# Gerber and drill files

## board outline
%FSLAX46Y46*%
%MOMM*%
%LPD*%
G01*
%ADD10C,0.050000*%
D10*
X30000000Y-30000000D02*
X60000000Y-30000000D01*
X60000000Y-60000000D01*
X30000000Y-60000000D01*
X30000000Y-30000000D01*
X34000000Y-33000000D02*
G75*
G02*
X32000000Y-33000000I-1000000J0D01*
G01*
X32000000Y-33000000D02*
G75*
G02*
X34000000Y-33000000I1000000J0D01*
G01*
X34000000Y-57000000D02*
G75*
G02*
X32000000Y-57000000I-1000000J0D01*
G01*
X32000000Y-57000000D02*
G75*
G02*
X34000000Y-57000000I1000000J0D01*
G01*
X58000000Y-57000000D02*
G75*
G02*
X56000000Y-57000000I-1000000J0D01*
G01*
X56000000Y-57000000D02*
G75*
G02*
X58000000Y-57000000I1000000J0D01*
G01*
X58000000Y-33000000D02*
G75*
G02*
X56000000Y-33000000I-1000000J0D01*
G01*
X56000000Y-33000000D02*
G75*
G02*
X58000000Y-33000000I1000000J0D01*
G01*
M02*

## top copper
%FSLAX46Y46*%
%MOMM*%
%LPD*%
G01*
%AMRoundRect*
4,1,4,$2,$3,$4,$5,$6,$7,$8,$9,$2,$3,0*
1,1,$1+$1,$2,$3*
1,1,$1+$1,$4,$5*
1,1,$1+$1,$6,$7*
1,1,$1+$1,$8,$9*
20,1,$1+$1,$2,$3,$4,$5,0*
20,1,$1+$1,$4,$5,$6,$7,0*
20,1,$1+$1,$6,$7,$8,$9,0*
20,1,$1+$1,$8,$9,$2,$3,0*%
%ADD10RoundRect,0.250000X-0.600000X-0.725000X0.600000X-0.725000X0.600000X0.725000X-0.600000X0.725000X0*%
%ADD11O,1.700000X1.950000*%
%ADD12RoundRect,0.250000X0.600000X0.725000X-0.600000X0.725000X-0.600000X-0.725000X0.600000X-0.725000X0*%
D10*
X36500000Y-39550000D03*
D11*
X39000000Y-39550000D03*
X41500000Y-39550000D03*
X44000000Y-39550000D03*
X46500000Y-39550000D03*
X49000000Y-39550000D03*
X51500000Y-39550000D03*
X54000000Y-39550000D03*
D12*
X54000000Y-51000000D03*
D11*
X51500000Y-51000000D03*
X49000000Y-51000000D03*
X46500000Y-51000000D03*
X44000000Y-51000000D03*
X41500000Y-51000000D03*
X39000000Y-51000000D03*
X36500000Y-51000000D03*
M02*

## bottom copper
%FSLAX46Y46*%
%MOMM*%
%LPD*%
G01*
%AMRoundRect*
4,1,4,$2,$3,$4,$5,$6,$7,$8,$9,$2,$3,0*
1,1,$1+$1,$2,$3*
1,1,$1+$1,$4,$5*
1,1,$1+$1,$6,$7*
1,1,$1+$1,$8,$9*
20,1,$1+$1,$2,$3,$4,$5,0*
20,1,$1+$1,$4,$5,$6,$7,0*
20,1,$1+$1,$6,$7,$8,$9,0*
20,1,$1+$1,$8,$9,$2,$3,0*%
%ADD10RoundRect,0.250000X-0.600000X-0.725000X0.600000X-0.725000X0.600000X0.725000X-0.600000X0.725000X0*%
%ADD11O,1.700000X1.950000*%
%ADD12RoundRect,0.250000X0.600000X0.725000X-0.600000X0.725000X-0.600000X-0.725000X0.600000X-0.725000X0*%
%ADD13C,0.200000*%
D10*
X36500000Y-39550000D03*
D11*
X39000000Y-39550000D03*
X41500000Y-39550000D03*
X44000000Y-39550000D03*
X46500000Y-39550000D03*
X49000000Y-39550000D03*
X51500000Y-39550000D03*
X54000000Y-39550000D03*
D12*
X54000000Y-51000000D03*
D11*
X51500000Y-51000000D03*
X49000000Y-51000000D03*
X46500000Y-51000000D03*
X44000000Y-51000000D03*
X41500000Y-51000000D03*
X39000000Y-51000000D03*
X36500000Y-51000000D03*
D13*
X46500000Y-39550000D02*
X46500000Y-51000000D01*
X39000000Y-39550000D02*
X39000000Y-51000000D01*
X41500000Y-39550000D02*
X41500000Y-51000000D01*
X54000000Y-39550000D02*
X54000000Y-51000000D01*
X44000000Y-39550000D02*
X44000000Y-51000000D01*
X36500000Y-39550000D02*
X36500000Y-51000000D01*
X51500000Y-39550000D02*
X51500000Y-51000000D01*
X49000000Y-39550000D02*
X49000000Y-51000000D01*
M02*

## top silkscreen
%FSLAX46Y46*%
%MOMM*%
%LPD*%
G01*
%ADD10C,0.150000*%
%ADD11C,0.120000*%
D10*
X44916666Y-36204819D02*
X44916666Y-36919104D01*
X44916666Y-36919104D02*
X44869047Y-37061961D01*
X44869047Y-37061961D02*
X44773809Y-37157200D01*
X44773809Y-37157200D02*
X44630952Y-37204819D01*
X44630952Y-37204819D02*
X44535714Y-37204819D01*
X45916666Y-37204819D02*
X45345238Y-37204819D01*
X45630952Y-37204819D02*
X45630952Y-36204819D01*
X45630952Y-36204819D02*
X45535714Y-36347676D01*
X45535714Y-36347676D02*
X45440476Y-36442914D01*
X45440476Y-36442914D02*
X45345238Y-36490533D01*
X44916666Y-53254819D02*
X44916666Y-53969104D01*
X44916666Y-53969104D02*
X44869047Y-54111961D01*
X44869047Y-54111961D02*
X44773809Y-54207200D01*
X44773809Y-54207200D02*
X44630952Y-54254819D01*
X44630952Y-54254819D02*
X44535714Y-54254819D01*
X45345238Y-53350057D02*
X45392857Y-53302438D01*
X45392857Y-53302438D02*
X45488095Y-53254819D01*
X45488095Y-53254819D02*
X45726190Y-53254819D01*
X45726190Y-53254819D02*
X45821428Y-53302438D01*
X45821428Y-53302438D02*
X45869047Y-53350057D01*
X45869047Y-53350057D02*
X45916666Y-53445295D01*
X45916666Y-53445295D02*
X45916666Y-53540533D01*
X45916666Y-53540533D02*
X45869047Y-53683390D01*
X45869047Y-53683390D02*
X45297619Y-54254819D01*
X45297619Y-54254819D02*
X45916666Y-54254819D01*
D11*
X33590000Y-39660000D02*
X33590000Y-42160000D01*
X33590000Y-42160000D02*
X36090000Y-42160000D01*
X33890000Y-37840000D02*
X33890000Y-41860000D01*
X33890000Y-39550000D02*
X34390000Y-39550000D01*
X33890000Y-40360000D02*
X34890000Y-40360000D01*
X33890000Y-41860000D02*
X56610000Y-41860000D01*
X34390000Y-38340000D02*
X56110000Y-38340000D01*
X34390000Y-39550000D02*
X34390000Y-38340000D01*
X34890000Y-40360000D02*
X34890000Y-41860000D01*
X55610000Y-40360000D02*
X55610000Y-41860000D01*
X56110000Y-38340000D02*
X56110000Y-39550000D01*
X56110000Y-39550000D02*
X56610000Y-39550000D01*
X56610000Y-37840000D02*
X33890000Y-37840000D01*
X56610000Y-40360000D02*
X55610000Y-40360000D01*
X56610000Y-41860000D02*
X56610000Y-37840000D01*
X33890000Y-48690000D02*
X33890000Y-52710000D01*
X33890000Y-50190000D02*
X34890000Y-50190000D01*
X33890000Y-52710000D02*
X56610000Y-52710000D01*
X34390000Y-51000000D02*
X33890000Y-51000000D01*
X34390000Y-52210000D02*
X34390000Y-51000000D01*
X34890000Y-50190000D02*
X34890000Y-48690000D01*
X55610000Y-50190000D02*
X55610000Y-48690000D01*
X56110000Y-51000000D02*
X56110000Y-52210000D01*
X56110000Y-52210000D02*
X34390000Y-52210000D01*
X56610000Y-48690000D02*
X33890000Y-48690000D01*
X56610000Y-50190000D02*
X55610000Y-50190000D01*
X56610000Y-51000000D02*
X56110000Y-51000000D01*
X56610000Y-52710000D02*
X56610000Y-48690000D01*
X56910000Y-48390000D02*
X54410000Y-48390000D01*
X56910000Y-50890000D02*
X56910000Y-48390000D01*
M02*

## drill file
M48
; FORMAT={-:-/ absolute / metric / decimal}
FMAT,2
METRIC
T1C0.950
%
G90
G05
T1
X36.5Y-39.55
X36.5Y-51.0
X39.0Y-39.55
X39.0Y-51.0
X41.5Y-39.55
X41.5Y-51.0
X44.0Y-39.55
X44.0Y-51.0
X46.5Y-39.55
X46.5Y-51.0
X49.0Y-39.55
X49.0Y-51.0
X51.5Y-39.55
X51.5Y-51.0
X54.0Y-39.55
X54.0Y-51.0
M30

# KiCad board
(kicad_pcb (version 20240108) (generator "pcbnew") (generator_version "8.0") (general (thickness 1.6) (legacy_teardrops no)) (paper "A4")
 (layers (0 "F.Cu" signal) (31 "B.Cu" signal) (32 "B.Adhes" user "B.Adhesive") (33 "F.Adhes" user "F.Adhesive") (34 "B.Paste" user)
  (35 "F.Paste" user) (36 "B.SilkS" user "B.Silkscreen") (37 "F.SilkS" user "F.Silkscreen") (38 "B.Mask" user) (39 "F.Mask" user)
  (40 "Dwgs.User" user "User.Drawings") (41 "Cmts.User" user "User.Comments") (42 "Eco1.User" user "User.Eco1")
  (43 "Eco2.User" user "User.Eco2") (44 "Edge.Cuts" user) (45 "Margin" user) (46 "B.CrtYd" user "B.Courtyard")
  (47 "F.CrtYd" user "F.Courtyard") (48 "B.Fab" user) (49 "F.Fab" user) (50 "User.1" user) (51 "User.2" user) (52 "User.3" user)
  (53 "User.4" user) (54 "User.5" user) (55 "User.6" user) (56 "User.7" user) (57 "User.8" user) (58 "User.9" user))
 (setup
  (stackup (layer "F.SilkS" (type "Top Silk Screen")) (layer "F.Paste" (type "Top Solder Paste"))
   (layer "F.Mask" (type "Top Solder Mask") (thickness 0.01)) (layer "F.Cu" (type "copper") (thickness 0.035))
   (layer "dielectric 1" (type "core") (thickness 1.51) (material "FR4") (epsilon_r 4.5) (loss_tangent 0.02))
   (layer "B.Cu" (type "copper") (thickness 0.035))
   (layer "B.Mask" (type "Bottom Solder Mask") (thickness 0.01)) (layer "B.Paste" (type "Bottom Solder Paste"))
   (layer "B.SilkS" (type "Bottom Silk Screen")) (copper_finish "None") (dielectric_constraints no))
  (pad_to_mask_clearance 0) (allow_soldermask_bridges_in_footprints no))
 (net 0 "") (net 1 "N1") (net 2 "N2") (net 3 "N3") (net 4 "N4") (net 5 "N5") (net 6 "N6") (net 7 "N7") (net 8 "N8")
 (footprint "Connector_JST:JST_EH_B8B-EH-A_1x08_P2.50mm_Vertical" (layer "F.Cu") (at 36.5 39.55)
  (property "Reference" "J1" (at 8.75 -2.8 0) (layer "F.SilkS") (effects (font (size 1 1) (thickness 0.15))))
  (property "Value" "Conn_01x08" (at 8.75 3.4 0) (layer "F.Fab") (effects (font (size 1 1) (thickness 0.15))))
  (fp_line (start -2.91 0.11) (end -2.91 2.61) (stroke (width 0.12) (type solid)) (layer "F.SilkS"))
  (fp_line (start -2.91 2.61) (end -0.41 2.61) (stroke (width 0.12) (type solid)) (layer "F.SilkS"))
  (fp_line (start -2.61 -1.71) (end -2.61 2.31) (stroke (width 0.12) (type solid)) (layer "F.SilkS"))
  (fp_line (start -2.61 0) (end -2.11 0) (stroke (width 0.12) (type solid)) (layer "F.SilkS"))
  (fp_line (start -2.61 0.81) (end -1.61 0.81) (stroke (width 0.12) (type solid)) (layer "F.SilkS"))
  (fp_line (start -2.61 2.31) (end 20.11 2.31) (stroke (width 0.12) (type solid)) (layer "F.SilkS"))
  (fp_line (start -2.11 -1.21) (end 19.61 -1.21) (stroke (width 0.12) (type solid)) (layer "F.SilkS"))
  (fp_line (start -2.11 0) (end -2.11 -1.21) (stroke (width 0.12) (type solid)) (layer "F.SilkS"))
  (fp_line (start -1.61 0.81) (end -1.61 2.31) (stroke (width 0.12) (type solid)) (layer "F.SilkS"))
  (fp_line (start 19.11 0.81) (end 19.11 2.31) (stroke (width 0.12) (type solid)) (layer "F.SilkS"))
  (fp_line (start 19.61 -1.21) (end 19.61 0) (stroke (width 0.12) (type solid)) (layer "F.SilkS"))
  (fp_line (start 19.61 0) (end 20.11 0) (stroke (width 0.12) (type solid)) (layer "F.SilkS"))
  (fp_line (start 20.11 -1.71) (end -2.61 -1.71) (stroke (width 0.12) (type solid)) (layer "F.SilkS"))
  (fp_line (start 20.11 0.81) (end 19.11 0.81) (stroke (width 0.12) (type solid)) (layer "F.SilkS"))
  (fp_line (start 20.11 2.31) (end 20.11 -1.71) (stroke (width 0.12) (type solid)) (layer "F.SilkS"))
  (pad "1" thru_hole roundrect (at 0 0) (size 1.7 1.95) (drill 0.95) (layers "*.Cu" "*.Mask") (remove_unused_layers no)
   (roundrect_rratio 0.147059) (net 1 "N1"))
  (pad "2" thru_hole oval (at 2.5 0) (size 1.7 1.95) (drill 0.95) (layers "*.Cu" "*.Mask") (remove_unused_layers no) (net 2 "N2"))
  (pad "3" thru_hole oval (at 5 0) (size 1.7 1.95) (drill 0.95) (layers "*.Cu" "*.Mask") (remove_unused_layers no) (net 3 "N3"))
  (pad "4" thru_hole oval (at 7.5 0) (size 1.7 1.95) (drill 0.95) (layers "*.Cu" "*.Mask") (remove_unused_layers no) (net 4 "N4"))
  (pad "5" thru_hole oval (at 10 0) (size 1.7 1.95) (drill 0.95) (layers "*.Cu" "*.Mask") (remove_unused_layers no) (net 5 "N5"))
  (pad "6" thru_hole oval (at 12.5 0) (size 1.7 1.95) (drill 0.95) (layers "*.Cu" "*.Mask") (remove_unused_layers no) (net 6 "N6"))
  (pad "7" thru_hole oval (at 15 0) (size 1.7 1.95) (drill 0.95) (layers "*.Cu" "*.Mask") (remove_unused_layers no) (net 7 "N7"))
  (pad "8" thru_hole oval (at 17.5 0) (size 1.7 1.95) (drill 0.95) (layers "*.Cu" "*.Mask") (remove_unused_layers no) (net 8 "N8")))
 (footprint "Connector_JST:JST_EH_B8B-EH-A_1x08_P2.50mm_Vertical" (layer "F.Cu") (at 54 51 180)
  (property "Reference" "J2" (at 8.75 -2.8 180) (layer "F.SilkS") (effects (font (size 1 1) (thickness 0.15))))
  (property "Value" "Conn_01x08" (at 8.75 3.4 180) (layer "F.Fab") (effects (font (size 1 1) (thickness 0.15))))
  (fp_line (start 20.11 2.31) (end 20.11 -1.71) (stroke (width 0.12) (type solid)) (layer "F.SilkS"))
  (fp_line (start 20.11 0.81) (end 19.11 0.81) (stroke (width 0.12) (type solid)) (layer "F.SilkS"))
  (fp_line (start 20.11 -1.71) (end -2.61 -1.71) (stroke (width 0.12) (type solid)) (layer "F.SilkS"))
  (fp_line (start 19.61 0) (end 20.11 0) (stroke (width 0.12) (type solid)) (layer "F.SilkS"))
  (fp_line (start 19.61 -1.21) (end 19.61 0) (stroke (width 0.12) (type solid)) (layer "F.SilkS"))
  (fp_line (start 19.11 0.81) (end 19.11 2.31) (stroke (width 0.12) (type solid)) (layer "F.SilkS"))
  (fp_line (start -1.61 0.81) (end -1.61 2.31) (stroke (width 0.12) (type solid)) (layer "F.SilkS"))
  (fp_line (start -2.11 0) (end -2.11 -1.21) (stroke (width 0.12) (type solid)) (layer "F.SilkS"))
  (fp_line (start -2.11 -1.21) (end 19.61 -1.21) (stroke (width 0.12) (type solid)) (layer "F.SilkS"))
  (fp_line (start -2.61 2.31) (end 20.11 2.31) (stroke (width 0.12) (type solid)) (layer "F.SilkS"))
  (fp_line (start -2.61 0.81) (end -1.61 0.81) (stroke (width 0.12) (type solid)) (layer "F.SilkS"))
  (fp_line (start -2.61 0) (end -2.11 0) (stroke (width 0.12) (type solid)) (layer "F.SilkS"))
  (fp_line (start -2.61 -1.71) (end -2.61 2.31) (stroke (width 0.12) (type solid)) (layer "F.SilkS"))
  (fp_line (start -2.91 2.61) (end -0.41 2.61) (stroke (width 0.12) (type solid)) (layer "F.SilkS"))
  (fp_line (start -2.91 0.11) (end -2.91 2.61) (stroke (width 0.12) (type solid)) (layer "F.SilkS"))
  (pad "1" thru_hole roundrect (at 0 0 180) (size 1.7 1.95) (drill 0.95) (layers "*.Cu" "*.Mask") (remove_unused_layers no)
   (roundrect_rratio 0.147059) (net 8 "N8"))
  (pad "2" thru_hole oval (at 2.5 0 180) (size 1.7 1.95) (drill 0.95) (layers "*.Cu" "*.Mask") (remove_unused_layers no) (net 7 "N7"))
  (pad "3" thru_hole oval (at 5 0 180) (size 1.7 1.95) (drill 0.95) (layers "*.Cu" "*.Mask") (remove_unused_layers no) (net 6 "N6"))
  (pad "4" thru_hole oval (at 7.5 0 180) (size 1.7 1.95) (drill 0.95) (layers "*.Cu" "*.Mask") (remove_unused_layers no) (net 5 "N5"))
  (pad "5" thru_hole oval (at 10 0 180) (size 1.7 1.95) (drill 0.95) (layers "*.Cu" "*.Mask") (remove_unused_layers no) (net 4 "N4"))
  (pad "6" thru_hole oval (at 12.5 0 180) (size 1.7 1.95) (drill 0.95) (layers "*.Cu" "*.Mask") (remove_unused_layers no) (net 3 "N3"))
  (pad "7" thru_hole oval (at 15 0 180) (size 1.7 1.95) (drill 0.95) (layers "*.Cu" "*.Mask") (remove_unused_layers no) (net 2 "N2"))
  (pad "8" thru_hole oval (at 17.5 0 180) (size 1.7 1.95) (drill 0.95) (layers "*.Cu" "*.Mask") (remove_unused_layers no) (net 1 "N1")))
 (gr_rect (start 30 30) (end 60 60) (stroke (width 0.05) (type default)) (fill none) (layer "Edge.Cuts"))
 (gr_circle (center 33 33) (end 33 32) (stroke (width 0.05) (type default)) (fill none) (layer "Edge.Cuts"))
 (gr_circle (center 33 57) (end 33 58) (stroke (width 0.05) (type default)) (fill none) (layer "Edge.Cuts"))
 (gr_circle (center 57 57) (end 57 58) (stroke (width 0.05) (type default)) (fill none) (layer "Edge.Cuts"))
 (gr_circle (center 57 33) (end 57 32) (stroke (width 0.05) (type default)) (fill none) (layer "Edge.Cuts"))
 (segment (start 46.5 39.55) (end 46.5 51) (width 0.2) (layer "B.Cu") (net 5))
 (segment (start 39 39.55) (end 39 51) (width 0.2) (layer "B.Cu") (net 2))
 (segment (start 41.5 39.55) (end 41.5 51) (width 0.2) (layer "B.Cu") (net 3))
 (segment (start 54 39.55) (end 54 51) (width 0.2) (layer "B.Cu") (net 8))
 (segment (start 44 39.55) (end 44 51) (width 0.2) (layer "B.Cu") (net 4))
 (segment (start 36.5 39.55) (end 36.5 51) (width 0.2) (layer "B.Cu") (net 1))
 (segment (start 51.5 39.55) (end 51.5 51) (width 0.2) (layer "B.Cu") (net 7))
 (segment (start 49 39.55) (end 49 51) (width 0.2) (layer "B.Cu") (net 6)))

